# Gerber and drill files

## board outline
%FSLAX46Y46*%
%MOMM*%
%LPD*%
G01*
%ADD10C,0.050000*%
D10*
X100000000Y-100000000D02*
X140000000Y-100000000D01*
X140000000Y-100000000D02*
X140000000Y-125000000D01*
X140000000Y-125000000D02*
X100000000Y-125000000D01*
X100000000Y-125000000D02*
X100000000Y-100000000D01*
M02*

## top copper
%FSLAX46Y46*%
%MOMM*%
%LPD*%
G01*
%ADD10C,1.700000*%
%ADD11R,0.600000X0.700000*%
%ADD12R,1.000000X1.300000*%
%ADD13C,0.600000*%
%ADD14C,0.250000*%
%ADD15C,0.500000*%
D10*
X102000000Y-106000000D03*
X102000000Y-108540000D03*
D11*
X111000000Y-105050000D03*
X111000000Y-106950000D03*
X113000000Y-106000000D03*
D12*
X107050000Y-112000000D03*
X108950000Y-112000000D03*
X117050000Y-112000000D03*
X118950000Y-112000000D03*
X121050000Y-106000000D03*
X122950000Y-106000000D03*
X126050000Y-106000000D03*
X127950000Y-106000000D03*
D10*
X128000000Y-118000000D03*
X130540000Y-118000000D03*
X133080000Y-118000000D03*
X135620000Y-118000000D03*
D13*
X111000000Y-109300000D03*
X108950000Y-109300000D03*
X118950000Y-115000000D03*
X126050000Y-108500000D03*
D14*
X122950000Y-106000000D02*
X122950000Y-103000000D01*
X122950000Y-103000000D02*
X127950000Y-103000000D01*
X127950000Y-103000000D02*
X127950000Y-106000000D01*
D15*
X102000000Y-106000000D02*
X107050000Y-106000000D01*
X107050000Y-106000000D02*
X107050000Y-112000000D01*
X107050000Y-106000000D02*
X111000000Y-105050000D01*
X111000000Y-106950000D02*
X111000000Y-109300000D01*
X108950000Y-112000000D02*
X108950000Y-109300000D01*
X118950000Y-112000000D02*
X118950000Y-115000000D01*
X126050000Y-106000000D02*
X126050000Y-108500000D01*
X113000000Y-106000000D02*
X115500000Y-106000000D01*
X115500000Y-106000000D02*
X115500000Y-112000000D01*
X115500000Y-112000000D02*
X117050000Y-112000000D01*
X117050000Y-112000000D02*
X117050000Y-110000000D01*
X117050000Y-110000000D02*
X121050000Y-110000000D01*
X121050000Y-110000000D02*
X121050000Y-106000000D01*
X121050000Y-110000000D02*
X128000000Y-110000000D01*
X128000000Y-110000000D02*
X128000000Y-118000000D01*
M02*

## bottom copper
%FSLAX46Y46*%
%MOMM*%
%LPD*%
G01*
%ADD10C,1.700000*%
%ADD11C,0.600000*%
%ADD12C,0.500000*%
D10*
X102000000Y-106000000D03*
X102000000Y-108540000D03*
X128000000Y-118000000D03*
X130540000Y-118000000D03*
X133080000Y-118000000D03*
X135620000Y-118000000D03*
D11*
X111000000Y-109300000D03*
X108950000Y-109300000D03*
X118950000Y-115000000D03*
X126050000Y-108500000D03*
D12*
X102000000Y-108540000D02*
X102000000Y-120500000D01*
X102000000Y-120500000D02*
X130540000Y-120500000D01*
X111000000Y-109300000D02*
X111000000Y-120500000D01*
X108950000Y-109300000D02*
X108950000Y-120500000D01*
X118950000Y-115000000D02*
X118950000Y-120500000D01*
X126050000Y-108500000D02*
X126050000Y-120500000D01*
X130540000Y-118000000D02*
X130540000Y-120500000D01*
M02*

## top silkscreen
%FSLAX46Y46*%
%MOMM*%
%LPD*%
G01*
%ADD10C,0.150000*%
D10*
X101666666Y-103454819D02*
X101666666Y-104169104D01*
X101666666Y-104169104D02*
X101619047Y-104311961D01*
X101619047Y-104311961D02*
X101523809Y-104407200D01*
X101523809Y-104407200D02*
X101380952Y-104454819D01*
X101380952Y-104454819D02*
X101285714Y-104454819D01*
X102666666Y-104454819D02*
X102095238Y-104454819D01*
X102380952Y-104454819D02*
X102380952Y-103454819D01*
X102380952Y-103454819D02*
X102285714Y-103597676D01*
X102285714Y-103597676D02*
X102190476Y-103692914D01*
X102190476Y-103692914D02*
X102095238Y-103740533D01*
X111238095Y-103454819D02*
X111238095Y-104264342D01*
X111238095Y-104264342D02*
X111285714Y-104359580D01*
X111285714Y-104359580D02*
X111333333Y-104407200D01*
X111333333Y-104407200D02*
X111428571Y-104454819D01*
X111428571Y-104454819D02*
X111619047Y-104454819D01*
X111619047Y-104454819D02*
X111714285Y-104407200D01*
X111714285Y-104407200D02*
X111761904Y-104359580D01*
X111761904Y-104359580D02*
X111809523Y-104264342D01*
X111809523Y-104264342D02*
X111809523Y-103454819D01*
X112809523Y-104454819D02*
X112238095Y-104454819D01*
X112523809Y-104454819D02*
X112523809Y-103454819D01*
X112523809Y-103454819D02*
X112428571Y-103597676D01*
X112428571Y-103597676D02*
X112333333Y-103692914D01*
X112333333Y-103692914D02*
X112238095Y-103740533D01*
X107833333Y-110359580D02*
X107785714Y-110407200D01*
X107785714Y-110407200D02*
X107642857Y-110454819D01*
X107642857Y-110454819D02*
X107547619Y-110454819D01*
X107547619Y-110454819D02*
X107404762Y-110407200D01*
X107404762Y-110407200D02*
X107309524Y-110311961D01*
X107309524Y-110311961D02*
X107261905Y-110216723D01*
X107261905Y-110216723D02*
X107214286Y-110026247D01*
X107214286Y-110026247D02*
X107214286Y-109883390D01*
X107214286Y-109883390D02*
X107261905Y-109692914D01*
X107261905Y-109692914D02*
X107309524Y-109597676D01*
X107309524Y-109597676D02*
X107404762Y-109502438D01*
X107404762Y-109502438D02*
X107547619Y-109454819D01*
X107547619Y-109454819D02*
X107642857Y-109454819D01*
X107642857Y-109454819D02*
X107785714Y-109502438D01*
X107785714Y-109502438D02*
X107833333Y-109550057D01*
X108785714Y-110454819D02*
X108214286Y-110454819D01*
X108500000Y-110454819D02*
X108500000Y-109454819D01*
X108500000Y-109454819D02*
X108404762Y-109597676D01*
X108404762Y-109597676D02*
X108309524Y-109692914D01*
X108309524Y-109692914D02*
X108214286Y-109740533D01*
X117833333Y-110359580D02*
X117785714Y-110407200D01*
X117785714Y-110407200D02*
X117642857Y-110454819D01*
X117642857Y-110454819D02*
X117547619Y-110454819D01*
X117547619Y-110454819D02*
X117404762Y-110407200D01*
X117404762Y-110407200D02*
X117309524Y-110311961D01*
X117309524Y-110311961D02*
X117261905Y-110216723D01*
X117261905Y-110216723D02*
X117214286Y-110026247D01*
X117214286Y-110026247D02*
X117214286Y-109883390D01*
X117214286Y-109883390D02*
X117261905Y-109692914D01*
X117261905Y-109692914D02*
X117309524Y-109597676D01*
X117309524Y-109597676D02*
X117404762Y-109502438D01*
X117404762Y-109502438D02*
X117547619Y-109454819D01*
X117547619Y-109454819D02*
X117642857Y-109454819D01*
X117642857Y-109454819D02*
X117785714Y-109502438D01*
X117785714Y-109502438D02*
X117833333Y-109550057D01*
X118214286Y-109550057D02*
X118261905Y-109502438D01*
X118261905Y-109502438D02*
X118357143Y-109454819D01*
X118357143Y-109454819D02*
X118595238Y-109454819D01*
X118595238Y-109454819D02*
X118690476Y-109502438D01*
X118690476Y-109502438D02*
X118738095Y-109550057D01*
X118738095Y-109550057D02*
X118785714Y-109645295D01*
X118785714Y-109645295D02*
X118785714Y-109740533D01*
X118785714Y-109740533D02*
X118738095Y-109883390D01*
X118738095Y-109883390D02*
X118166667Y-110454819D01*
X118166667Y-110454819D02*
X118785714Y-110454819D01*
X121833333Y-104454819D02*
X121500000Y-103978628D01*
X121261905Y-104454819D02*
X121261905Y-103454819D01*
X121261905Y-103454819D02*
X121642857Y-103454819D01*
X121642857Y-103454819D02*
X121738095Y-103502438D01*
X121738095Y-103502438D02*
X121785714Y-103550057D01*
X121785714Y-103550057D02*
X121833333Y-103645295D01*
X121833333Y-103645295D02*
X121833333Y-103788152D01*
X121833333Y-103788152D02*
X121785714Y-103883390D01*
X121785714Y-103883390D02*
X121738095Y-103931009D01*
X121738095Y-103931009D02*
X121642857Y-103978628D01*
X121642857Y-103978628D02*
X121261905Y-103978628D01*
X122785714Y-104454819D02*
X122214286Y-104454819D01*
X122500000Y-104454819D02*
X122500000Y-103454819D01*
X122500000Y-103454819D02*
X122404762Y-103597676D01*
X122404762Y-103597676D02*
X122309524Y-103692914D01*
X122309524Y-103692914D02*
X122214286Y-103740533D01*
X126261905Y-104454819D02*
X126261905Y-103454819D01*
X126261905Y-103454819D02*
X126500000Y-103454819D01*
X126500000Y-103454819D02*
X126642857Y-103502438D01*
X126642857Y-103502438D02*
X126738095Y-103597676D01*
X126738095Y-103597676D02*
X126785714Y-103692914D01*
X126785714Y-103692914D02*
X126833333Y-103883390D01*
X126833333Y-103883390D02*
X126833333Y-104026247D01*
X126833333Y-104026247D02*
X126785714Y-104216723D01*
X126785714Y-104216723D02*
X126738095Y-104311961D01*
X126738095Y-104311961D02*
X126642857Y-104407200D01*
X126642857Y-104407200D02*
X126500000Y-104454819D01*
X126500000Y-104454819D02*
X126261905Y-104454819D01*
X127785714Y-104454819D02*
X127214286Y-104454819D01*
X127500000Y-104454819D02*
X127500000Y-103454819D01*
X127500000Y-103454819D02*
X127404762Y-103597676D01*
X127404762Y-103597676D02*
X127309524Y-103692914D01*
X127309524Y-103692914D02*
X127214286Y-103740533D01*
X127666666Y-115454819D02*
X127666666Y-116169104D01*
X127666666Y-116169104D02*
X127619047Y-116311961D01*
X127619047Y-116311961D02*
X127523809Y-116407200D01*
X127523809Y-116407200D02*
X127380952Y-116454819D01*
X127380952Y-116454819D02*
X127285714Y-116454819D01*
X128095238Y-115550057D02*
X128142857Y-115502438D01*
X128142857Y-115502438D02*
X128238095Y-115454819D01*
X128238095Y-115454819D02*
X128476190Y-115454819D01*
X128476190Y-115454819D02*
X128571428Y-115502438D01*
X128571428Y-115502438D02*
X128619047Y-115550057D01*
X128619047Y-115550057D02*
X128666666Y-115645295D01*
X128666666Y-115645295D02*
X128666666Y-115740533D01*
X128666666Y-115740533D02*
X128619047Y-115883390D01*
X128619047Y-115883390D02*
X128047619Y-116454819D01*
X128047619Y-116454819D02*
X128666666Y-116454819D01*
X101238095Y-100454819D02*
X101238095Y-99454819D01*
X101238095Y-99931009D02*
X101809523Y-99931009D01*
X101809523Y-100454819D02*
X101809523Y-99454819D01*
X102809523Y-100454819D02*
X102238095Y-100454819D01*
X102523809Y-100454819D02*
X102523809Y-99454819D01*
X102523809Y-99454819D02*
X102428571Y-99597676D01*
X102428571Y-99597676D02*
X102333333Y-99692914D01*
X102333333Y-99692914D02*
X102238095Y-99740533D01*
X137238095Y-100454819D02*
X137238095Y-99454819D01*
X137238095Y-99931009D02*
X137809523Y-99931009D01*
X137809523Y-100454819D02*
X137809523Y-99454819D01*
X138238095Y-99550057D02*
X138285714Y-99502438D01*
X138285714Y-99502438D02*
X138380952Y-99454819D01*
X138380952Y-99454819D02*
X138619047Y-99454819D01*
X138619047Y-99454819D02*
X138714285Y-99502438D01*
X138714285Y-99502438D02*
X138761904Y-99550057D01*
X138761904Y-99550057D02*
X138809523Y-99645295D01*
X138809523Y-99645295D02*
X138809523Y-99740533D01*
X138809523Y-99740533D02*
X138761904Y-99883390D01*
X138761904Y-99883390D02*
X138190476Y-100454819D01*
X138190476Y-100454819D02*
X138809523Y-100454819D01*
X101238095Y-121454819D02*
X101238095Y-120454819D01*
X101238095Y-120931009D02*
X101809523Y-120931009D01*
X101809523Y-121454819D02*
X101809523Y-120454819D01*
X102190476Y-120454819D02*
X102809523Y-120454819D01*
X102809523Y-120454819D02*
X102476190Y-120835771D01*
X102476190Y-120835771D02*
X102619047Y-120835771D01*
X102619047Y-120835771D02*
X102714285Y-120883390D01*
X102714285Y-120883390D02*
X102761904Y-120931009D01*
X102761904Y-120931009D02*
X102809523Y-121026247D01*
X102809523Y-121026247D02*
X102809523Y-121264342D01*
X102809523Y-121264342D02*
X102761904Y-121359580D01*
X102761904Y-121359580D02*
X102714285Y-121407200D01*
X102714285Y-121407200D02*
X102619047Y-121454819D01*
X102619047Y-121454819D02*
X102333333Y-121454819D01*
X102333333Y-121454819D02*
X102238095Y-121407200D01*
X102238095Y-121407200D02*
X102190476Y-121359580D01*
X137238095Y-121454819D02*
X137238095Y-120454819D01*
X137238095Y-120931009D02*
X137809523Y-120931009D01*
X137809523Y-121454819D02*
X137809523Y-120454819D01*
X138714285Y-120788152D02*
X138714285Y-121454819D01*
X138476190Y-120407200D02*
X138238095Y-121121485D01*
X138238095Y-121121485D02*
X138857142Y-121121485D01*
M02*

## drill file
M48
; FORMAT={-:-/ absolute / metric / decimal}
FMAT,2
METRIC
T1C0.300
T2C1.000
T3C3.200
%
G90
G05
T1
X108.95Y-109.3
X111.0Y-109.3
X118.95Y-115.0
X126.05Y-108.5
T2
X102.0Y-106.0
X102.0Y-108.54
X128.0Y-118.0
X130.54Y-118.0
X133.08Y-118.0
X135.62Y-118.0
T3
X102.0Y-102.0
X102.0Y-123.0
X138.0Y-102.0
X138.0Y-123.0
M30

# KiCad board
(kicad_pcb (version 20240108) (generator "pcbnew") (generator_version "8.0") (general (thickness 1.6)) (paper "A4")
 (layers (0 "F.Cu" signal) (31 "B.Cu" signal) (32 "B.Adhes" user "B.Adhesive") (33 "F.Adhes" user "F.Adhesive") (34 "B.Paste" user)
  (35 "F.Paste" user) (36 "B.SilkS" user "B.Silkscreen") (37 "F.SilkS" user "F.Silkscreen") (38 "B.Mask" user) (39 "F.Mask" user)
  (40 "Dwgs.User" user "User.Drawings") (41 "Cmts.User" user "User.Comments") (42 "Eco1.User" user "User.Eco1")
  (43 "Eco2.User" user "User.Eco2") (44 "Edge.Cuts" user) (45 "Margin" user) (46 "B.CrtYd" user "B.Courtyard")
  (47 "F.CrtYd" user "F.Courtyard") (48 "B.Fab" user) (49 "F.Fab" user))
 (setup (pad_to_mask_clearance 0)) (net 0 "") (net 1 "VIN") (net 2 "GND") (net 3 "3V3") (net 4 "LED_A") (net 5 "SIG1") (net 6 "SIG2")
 (gr_line (start 100 100) (end 140 100) (stroke (width 0.05) (type default)) (layer "Edge.Cuts"))
 (gr_line (start 140 100) (end 140 125) (stroke (width 0.05) (type default)) (layer "Edge.Cuts"))
 (gr_line (start 140 125) (end 100 125) (stroke (width 0.05) (type default)) (layer "Edge.Cuts"))
 (gr_line (start 100 125) (end 100 100) (stroke (width 0.05) (type default)) (layer "Edge.Cuts"))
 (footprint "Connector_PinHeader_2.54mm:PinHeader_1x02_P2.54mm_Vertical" (layer "F.Cu") (at 102 106)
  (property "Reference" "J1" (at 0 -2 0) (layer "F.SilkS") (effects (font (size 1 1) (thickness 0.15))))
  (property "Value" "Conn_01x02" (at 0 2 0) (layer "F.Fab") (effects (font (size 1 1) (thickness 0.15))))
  (pad "1" thru_hole circle (at 0 0) (size 1.7 1.7) (drill 1) (layers "*.Cu" "*.Mask") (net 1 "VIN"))
  (pad "2" thru_hole circle (at 0 2.54) (size 1.7 1.7) (drill 1) (layers "*.Cu" "*.Mask") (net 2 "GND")))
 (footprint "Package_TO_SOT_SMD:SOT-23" (layer "F.Cu") (at 112 106)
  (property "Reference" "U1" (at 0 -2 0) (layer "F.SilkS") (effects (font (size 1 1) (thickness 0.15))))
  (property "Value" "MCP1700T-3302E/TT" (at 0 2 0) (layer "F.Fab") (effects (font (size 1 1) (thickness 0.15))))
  (pad "1" smd rect (at -1 -0.95) (size 0.6 0.7) (layers "F.Cu" "F.Paste" "F.Mask") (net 1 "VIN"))
  (pad "2" smd rect (at -1 0.95) (size 0.6 0.7) (layers "F.Cu" "F.Paste" "F.Mask") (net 2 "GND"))
  (pad "3" smd rect (at 1 0) (size 0.6 0.7) (layers "F.Cu" "F.Paste" "F.Mask") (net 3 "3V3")))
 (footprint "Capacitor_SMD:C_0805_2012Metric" (layer "F.Cu") (at 108 112)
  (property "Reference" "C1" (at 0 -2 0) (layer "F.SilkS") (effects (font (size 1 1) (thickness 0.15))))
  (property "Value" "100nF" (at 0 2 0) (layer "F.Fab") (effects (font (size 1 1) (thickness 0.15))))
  (pad "1" smd rect (at -0.95 0) (size 1 1.3) (layers "F.Cu" "F.Paste" "F.Mask") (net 1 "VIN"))
  (pad "2" smd rect (at 0.95 0) (size 1 1.3) (layers "F.Cu" "F.Paste" "F.Mask") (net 2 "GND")))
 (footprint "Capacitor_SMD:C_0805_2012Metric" (layer "F.Cu") (at 118 112)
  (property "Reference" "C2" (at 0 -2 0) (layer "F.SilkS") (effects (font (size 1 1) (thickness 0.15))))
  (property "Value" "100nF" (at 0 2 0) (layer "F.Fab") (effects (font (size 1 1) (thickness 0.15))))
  (pad "1" smd rect (at -0.95 0) (size 1 1.3) (layers "F.Cu" "F.Paste" "F.Mask") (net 3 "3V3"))
  (pad "2" smd rect (at 0.95 0) (size 1 1.3) (layers "F.Cu" "F.Paste" "F.Mask") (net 2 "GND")))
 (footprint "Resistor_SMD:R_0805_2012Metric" (layer "F.Cu") (at 122 106)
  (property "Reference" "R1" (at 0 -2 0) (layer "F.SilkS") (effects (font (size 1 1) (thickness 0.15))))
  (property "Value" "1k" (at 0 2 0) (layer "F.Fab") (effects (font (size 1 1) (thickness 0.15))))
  (pad "1" smd rect (at -0.95 0) (size 1 1.3) (layers "F.Cu" "F.Paste" "F.Mask") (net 3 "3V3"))
  (pad "2" smd rect (at 0.95 0) (size 1 1.3) (layers "F.Cu" "F.Paste" "F.Mask") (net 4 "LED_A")))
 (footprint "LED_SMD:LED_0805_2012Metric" (layer "F.Cu") (at 127 106)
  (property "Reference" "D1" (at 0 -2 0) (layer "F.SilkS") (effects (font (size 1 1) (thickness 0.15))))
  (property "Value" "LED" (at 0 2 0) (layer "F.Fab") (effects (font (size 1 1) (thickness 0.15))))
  (pad "1" smd rect (at -0.95 0) (size 1 1.3) (layers "F.Cu" "F.Paste" "F.Mask") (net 2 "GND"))
  (pad "2" smd rect (at 0.95 0) (size 1 1.3) (layers "F.Cu" "F.Paste" "F.Mask") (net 4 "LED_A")))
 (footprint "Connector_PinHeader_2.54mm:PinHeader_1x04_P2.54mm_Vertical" (layer "F.Cu") (at 128 118)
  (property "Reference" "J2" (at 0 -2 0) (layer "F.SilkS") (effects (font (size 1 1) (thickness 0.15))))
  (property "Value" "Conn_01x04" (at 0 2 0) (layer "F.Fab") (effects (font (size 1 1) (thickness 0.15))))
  (pad "1" thru_hole circle (at 0 0) (size 1.7 1.7) (drill 1) (layers "*.Cu" "*.Mask") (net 3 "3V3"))
  (pad "2" thru_hole circle (at 2.54 0) (size 1.7 1.7) (drill 1) (layers "*.Cu" "*.Mask") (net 2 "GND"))
  (pad "3" thru_hole circle (at 5.08 0) (size 1.7 1.7) (drill 1) (layers "*.Cu" "*.Mask") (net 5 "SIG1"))
  (pad "4" thru_hole circle (at 7.62 0) (size 1.7 1.7) (drill 1) (layers "*.Cu" "*.Mask") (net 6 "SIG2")))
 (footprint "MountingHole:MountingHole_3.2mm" (layer "F.Cu") (at 102 102)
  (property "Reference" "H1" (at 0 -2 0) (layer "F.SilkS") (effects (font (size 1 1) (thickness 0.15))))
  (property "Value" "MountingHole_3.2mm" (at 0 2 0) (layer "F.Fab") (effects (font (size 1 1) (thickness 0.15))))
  (pad "1" np_thru_hole circle (at 0 0) (size 3.2 3.2) (drill 3.2) (layers "*.Cu" "*.Mask")))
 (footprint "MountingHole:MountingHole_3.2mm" (layer "F.Cu") (at 138 102)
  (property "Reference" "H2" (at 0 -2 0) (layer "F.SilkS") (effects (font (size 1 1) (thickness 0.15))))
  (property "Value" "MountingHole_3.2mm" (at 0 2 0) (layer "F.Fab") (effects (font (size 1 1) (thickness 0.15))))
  (pad "1" np_thru_hole circle (at 0 0) (size 3.2 3.2) (drill 3.2) (layers "*.Cu" "*.Mask")))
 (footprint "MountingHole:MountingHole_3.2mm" (layer "F.Cu") (at 102 123)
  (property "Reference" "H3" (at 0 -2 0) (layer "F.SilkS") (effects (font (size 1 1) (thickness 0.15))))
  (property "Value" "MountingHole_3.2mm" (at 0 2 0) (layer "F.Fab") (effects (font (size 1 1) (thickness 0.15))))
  (pad "1" np_thru_hole circle (at 0 0) (size 3.2 3.2) (drill 3.2) (layers "*.Cu" "*.Mask")))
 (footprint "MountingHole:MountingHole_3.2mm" (layer "F.Cu") (at 138 123)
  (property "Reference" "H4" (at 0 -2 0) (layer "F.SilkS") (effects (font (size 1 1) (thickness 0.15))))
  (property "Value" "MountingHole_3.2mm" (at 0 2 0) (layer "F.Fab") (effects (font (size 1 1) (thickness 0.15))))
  (pad "1" np_thru_hole circle (at 0 0) (size 3.2 3.2) (drill 3.2) (layers "*.Cu" "*.Mask")))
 (segment (start 122.95 106) (end 122.95 103) (width 0.25) (layer "F.Cu") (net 4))
 (segment (start 122.95 103) (end 127.95 103) (width 0.25) (layer "F.Cu") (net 4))
 (segment (start 127.95 103) (end 127.95 106) (width 0.25) (layer "F.Cu") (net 4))
 (segment (start 102 106) (end 107.05 106) (width 0.5) (layer "F.Cu") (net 1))
 (segment (start 107.05 106) (end 107.05 112) (width 0.5) (layer "F.Cu") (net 1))
 (segment (start 107.05 106) (end 111 105.05) (width 0.5) (layer "F.Cu") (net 1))
 (segment (start 111 106.95) (end 111 109.3) (width 0.5) (layer "F.Cu") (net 2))
 (segment (start 108.95 112) (end 108.95 109.3) (width 0.5) (layer "F.Cu") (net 2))
 (segment (start 118.95 112) (end 118.95 115) (width 0.5) (layer "F.Cu") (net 2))
 (segment (start 126.05 106) (end 126.05 108.5) (width 0.5) (layer "F.Cu") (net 2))
 (segment (start 113 106) (end 115.5 106) (width 0.5) (layer "F.Cu") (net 3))
 (segment (start 115.5 106) (end 115.5 112) (width 0.5) (layer "F.Cu") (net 3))
 (segment (start 115.5 112) (end 117.05 112) (width 0.5) (layer "F.Cu") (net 3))
 (segment (start 117.05 112) (end 117.05 110) (width 0.5) (layer "F.Cu") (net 3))
 (segment (start 117.05 110) (end 121.05 110) (width 0.5) (layer "F.Cu") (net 3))
 (segment (start 121.05 110) (end 121.05 106) (width 0.5) (layer "F.Cu") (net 3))
 (segment (start 121.05 110) (end 128 110) (width 0.5) (layer "F.Cu") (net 3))
 (segment (start 128 110) (end 128 118) (width 0.5) (layer "F.Cu") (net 3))
 (segment (start 102 108.54) (end 102 120.5) (width 0.5) (layer "B.Cu") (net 2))
 (segment (start 102 120.5) (end 130.54 120.5) (width 0.5) (layer "B.Cu") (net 2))
 (segment (start 111 109.3) (end 111 120.5) (width 0.5) (layer "B.Cu") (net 2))
 (segment (start 108.95 109.3) (end 108.95 120.5) (width 0.5) (layer "B.Cu") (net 2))
 (segment (start 118.95 115) (end 118.95 120.5) (width 0.5) (layer "B.Cu") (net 2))
 (segment (start 126.05 108.5) (end 126.05 120.5) (width 0.5) (layer "B.Cu") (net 2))
 (segment (start 130.54 118) (end 130.54 120.5) (width 0.5) (layer "B.Cu") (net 2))
 (via (at 111 109.3) (size 0.6) (drill 0.3) (layers "F.Cu" "B.Cu") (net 2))
 (via (at 108.95 109.3) (size 0.6) (drill 0.3) (layers "F.Cu" "B.Cu") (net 2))
 (via (at 118.95 115) (size 0.6) (drill 0.3) (layers "F.Cu" "B.Cu") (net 2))
 (via (at 126.05 108.5) (size 0.6) (drill 0.3) (layers "F.Cu" "B.Cu") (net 2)))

